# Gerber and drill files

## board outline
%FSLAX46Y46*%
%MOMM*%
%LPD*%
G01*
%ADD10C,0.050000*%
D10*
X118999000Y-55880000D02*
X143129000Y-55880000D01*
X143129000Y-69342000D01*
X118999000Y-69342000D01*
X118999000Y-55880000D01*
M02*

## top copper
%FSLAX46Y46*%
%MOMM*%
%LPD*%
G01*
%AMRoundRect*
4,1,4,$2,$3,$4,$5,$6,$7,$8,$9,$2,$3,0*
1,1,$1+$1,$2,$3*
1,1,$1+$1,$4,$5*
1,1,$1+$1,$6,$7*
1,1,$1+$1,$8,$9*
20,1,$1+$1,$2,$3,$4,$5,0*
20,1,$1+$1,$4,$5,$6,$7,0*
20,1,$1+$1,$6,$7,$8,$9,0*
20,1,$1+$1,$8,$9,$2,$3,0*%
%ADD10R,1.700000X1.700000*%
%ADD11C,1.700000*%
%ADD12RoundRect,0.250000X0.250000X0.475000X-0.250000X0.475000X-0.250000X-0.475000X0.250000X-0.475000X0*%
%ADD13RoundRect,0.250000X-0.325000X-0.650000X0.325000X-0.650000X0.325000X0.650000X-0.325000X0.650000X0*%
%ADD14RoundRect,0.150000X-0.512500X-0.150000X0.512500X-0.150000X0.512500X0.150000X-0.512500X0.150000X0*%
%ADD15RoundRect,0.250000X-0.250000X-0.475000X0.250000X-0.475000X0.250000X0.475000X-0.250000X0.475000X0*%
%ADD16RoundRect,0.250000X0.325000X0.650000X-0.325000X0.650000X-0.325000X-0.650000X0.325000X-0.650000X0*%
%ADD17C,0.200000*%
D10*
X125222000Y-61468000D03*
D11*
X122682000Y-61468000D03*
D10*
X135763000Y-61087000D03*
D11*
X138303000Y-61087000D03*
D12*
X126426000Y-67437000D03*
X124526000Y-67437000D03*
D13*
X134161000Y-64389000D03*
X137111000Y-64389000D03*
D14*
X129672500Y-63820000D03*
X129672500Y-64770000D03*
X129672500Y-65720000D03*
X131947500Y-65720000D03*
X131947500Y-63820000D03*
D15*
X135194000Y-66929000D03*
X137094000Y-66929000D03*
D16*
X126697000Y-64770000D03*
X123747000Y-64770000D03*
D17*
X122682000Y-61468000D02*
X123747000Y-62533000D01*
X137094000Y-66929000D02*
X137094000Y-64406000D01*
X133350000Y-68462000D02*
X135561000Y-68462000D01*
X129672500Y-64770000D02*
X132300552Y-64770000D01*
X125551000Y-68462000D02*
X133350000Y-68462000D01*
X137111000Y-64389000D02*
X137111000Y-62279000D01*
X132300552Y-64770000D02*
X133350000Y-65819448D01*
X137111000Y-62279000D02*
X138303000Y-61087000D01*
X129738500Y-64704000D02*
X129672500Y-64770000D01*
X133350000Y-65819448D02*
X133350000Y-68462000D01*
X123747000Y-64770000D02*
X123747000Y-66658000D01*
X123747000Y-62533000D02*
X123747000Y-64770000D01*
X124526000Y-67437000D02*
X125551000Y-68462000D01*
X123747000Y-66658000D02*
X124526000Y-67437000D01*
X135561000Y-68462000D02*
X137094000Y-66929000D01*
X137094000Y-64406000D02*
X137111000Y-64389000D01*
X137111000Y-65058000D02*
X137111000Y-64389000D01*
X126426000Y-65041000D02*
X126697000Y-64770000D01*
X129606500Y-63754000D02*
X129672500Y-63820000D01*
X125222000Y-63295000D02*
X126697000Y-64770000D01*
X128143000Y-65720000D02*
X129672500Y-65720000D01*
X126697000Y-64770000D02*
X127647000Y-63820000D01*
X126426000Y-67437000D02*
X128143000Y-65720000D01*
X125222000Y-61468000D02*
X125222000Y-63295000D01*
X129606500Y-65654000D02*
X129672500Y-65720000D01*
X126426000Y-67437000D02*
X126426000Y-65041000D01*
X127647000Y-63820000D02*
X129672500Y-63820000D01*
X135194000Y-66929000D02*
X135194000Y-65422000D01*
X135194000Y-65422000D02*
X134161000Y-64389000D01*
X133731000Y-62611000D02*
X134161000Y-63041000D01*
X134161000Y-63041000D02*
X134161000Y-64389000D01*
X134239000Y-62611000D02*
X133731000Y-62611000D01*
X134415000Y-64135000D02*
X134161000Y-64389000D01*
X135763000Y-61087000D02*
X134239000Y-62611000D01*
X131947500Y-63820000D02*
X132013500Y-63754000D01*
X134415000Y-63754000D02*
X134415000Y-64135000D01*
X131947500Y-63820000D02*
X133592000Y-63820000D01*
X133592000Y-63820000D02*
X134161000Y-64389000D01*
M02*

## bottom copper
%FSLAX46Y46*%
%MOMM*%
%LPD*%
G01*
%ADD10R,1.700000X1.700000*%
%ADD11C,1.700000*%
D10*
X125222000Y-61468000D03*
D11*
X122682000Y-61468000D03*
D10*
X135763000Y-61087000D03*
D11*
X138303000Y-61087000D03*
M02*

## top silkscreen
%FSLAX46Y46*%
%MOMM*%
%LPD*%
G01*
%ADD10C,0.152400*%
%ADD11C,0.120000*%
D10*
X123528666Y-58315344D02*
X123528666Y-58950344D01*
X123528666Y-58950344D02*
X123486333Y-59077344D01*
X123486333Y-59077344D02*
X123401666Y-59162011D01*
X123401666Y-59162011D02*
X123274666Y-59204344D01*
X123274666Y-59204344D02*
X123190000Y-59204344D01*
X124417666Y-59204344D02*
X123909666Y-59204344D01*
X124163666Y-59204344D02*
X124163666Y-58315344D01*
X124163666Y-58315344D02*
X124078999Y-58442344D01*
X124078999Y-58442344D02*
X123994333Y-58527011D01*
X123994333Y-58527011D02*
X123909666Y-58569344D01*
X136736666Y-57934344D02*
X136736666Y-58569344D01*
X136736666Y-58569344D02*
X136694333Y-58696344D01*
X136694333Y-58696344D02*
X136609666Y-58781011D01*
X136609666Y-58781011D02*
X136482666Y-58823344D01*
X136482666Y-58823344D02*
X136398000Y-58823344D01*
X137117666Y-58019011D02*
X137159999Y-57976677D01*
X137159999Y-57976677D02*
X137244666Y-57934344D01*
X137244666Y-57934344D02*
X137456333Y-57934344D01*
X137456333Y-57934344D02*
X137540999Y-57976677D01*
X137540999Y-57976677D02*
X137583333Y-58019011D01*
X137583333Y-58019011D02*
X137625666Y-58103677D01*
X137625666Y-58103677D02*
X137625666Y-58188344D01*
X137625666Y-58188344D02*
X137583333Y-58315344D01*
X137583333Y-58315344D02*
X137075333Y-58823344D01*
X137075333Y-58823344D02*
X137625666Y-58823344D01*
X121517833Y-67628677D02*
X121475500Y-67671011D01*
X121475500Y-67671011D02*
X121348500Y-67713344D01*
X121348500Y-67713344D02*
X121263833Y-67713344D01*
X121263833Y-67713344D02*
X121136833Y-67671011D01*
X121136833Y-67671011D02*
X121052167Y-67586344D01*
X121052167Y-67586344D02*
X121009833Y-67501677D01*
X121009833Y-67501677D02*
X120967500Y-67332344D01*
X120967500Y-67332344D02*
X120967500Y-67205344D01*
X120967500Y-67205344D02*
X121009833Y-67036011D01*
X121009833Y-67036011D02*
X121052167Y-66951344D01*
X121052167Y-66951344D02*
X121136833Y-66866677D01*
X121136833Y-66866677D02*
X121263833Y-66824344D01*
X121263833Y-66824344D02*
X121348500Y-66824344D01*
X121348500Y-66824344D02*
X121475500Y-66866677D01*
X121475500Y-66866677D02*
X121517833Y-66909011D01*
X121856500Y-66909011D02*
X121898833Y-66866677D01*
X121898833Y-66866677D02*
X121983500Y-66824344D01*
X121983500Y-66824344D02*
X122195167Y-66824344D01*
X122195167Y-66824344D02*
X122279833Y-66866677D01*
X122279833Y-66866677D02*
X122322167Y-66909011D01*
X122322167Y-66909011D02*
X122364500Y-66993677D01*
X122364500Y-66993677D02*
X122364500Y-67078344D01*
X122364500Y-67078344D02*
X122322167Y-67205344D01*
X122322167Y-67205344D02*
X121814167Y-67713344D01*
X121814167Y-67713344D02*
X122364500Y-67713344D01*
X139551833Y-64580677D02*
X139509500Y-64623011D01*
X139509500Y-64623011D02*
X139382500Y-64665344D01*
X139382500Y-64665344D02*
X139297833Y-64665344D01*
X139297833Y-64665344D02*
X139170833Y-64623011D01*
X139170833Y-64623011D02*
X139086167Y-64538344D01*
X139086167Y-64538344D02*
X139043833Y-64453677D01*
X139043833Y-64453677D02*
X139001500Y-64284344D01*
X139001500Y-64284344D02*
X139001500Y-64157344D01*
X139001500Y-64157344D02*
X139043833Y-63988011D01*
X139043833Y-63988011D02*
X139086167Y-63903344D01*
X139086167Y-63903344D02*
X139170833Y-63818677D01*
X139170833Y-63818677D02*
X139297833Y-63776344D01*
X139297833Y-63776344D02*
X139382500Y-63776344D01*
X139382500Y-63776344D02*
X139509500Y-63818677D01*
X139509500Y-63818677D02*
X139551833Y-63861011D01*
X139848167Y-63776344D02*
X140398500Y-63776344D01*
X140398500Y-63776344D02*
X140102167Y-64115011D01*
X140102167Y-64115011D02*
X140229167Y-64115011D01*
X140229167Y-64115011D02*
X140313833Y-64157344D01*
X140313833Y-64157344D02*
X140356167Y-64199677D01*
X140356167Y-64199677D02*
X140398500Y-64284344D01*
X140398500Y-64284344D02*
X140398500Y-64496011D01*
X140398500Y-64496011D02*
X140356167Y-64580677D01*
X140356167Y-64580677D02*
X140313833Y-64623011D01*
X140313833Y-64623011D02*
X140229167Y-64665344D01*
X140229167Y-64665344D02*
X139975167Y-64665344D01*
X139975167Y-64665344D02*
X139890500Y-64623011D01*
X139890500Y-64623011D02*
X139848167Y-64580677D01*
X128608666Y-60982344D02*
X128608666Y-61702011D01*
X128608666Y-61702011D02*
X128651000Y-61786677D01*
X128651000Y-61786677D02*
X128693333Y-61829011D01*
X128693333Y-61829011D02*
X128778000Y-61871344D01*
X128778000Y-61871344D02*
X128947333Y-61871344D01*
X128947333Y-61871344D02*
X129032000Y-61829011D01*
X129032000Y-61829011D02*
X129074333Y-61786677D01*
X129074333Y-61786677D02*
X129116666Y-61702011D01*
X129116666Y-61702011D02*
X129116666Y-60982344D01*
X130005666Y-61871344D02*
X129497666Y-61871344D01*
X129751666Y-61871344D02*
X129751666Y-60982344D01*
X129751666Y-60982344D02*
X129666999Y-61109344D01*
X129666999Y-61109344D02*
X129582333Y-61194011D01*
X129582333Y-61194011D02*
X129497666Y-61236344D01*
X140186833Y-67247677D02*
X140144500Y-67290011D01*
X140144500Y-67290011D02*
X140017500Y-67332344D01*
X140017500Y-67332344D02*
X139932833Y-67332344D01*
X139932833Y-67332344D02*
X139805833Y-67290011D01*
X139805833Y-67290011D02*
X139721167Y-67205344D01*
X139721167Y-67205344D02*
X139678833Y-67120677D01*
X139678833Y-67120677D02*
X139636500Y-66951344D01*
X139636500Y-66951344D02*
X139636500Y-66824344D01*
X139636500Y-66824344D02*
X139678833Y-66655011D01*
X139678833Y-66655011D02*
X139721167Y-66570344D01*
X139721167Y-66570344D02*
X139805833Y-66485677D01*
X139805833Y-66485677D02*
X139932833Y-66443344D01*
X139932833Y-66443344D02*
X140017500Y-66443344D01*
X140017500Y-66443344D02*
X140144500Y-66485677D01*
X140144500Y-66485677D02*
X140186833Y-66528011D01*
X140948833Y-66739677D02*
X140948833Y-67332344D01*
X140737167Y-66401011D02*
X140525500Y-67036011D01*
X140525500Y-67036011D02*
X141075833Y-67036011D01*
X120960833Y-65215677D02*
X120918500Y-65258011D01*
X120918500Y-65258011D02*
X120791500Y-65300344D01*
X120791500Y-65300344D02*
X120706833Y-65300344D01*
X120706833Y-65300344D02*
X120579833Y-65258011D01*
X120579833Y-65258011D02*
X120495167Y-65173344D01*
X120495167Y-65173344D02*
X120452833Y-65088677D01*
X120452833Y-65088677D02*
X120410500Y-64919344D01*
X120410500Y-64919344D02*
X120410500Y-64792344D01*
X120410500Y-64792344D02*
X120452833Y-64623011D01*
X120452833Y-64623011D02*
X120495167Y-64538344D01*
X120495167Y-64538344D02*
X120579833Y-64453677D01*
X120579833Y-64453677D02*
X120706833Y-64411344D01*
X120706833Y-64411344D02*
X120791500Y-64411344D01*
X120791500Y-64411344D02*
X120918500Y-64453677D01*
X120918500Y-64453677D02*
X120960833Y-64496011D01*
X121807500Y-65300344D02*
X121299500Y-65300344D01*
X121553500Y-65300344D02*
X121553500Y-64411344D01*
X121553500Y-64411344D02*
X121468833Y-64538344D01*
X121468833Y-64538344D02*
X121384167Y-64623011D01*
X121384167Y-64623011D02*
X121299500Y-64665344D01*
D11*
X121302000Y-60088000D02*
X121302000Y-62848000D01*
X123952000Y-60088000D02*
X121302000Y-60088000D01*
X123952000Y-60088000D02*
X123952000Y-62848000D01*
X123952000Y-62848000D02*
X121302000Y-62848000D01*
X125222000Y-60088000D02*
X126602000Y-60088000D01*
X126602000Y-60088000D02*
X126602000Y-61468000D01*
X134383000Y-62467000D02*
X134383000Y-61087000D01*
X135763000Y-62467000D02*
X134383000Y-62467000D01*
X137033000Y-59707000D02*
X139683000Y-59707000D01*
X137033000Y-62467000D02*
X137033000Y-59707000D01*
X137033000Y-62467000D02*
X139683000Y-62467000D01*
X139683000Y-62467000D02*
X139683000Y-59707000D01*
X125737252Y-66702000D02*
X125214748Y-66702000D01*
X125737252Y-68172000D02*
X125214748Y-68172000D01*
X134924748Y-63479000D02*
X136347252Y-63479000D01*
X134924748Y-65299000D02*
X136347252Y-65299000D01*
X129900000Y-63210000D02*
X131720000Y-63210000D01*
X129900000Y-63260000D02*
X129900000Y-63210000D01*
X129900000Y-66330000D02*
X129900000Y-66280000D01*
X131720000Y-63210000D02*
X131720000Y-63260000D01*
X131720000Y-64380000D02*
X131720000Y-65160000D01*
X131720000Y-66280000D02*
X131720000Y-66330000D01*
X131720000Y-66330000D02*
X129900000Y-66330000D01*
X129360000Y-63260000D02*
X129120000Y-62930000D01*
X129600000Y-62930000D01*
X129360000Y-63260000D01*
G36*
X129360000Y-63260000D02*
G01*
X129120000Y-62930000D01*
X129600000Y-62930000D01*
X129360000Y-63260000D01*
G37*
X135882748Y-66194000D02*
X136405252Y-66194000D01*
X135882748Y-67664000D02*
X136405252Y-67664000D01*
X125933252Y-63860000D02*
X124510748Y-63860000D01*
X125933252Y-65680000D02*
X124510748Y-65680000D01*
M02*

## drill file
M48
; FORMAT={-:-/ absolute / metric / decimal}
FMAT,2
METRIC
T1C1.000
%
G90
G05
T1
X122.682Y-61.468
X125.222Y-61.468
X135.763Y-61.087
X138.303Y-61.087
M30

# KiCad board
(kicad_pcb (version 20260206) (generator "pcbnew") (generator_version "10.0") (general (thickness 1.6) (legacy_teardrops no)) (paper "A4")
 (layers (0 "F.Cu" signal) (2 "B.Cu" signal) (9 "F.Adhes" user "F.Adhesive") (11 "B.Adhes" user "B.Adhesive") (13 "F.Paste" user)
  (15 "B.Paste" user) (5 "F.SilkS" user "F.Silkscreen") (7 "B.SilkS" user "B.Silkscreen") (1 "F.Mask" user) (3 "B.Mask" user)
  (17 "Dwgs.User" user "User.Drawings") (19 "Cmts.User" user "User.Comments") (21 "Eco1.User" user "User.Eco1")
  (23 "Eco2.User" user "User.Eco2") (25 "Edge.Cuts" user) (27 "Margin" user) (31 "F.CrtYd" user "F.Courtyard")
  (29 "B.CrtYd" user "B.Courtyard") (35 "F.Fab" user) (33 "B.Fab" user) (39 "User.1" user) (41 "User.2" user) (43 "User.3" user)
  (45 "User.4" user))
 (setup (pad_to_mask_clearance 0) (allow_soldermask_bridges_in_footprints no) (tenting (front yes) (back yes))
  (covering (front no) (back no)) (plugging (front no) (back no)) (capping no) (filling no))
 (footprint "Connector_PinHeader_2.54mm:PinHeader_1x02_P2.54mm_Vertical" (layer "F.Cu") (at 125.222 61.468 -90)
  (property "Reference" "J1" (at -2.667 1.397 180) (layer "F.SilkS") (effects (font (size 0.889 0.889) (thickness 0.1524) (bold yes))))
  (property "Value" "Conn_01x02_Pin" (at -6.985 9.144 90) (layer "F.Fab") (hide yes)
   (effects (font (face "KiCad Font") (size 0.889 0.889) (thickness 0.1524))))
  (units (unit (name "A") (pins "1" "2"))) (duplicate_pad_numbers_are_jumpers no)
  (fp_line (start -1.38 3.92) (end 1.38 3.92) (stroke (width 0.12) (type solid)) (layer "F.SilkS"))
  (fp_line (start -1.38 1.27) (end -1.38 3.92) (stroke (width 0.12) (type solid)) (layer "F.SilkS"))
  (fp_line (start -1.38 1.27) (end 1.38 1.27) (stroke (width 0.12) (type solid)) (layer "F.SilkS"))
  (fp_line (start 1.38 1.27) (end 1.38 3.92) (stroke (width 0.12) (type solid)) (layer "F.SilkS"))
  (fp_line (start -1.38 0) (end -1.38 -1.38) (stroke (width 0.12) (type solid)) (layer "F.SilkS"))
  (fp_line (start -1.38 -1.38) (end 0 -1.38) (stroke (width 0.12) (type solid)) (layer "F.SilkS"))
  (pad "1" thru_hole rect (at 0 0 270) (size 1.7 1.7) (drill 1) (layers "*.Cu" "*.Mask") (remove_unused_layers no) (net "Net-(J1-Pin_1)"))
  (pad "2" thru_hole circle (at 0 2.54 270) (size 1.7 1.7) (drill 1) (layers "*.Cu" "*.Mask") (remove_unused_layers no) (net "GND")))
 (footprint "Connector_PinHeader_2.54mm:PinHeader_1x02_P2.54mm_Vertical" (layer "F.Cu") (at 135.763 61.087 90)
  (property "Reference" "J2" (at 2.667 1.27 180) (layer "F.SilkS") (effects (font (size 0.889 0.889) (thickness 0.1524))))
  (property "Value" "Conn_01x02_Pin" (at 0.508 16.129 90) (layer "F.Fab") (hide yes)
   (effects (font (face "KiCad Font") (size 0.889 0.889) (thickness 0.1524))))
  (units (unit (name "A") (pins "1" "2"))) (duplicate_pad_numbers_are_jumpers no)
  (fp_line (start -1.38 -1.38) (end 0 -1.38) (stroke (width 0.12) (type solid)) (layer "F.SilkS"))
  (fp_line (start -1.38 0) (end -1.38 -1.38) (stroke (width 0.12) (type solid)) (layer "F.SilkS"))
  (fp_line (start 1.38 1.27) (end 1.38 3.92) (stroke (width 0.12) (type solid)) (layer "F.SilkS"))
  (fp_line (start -1.38 1.27) (end 1.38 1.27) (stroke (width 0.12) (type solid)) (layer "F.SilkS"))
  (fp_line (start -1.38 1.27) (end -1.38 3.92) (stroke (width 0.12) (type solid)) (layer "F.SilkS"))
  (fp_line (start -1.38 3.92) (end 1.38 3.92) (stroke (width 0.12) (type solid)) (layer "F.SilkS"))
  (pad "1" thru_hole rect (at 0 0 90) (size 1.7 1.7) (drill 1) (layers "*.Cu" "*.Mask") (remove_unused_layers no) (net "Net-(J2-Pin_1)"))
  (pad "2" thru_hole circle (at 0 2.54 90) (size 1.7 1.7) (drill 1) (layers "*.Cu" "*.Mask") (remove_unused_layers no) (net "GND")))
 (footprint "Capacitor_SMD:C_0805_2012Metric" (layer "F.Cu") (at 125.476 67.437 180)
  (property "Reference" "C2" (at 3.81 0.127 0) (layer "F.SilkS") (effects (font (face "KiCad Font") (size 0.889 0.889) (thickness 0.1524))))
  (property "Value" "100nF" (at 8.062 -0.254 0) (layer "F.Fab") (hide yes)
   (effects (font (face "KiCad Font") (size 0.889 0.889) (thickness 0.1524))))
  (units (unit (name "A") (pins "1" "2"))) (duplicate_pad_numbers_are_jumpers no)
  (fp_line (start -0.261252 0.735) (end 0.261252 0.735) (stroke (width 0.12) (type solid)) (layer "F.SilkS"))
  (fp_line (start -0.261252 -0.735) (end 0.261252 -0.735) (stroke (width 0.12) (type solid)) (layer "F.SilkS"))
  (pad "1" smd roundrect (at -0.95 0 180) (size 1 1.45) (layers "F.Cu" "F.Mask" "F.Paste") (roundrect_rratio 0.25) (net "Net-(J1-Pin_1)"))
  (pad "2" smd roundrect (at 0.95 0 180) (size 1 1.45) (layers "F.Cu" "F.Mask" "F.Paste") (roundrect_rratio 0.25) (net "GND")))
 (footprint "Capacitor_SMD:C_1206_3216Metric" (layer "F.Cu") (at 135.636 64.389)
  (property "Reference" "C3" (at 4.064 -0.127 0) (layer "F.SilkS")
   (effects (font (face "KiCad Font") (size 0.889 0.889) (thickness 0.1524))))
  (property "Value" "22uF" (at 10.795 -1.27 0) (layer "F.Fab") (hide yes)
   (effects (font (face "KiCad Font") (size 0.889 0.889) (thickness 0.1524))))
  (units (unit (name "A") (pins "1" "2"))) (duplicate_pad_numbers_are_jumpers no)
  (fp_line (start -0.711252 -0.91) (end 0.711252 -0.91) (stroke (width 0.12) (type solid)) (layer "F.SilkS"))
  (fp_line (start -0.711252 0.91) (end 0.711252 0.91) (stroke (width 0.12) (type solid)) (layer "F.SilkS"))
  (pad "1" smd roundrect (at -1.475 0) (size 1.15 1.8) (layers "F.Cu" "F.Mask" "F.Paste") (roundrect_rratio 0.217391) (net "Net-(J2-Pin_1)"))
  (pad "2" smd roundrect (at 1.475 0) (size 1.15 1.8) (layers "F.Cu" "F.Mask" "F.Paste") (roundrect_rratio 0.217391) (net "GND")))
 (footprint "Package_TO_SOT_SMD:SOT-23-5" (layer "F.Cu") (at 130.81 64.77)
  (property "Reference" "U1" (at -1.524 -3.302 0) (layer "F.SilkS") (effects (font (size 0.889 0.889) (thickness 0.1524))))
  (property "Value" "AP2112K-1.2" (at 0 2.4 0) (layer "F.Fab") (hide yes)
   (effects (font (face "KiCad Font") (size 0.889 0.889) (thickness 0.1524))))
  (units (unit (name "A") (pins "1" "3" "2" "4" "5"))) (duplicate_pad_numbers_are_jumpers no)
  (fp_line (start -0.91 -1.56) (end 0.91 -1.56) (stroke (width 0.12) (type solid)) (layer "F.SilkS"))
  (fp_line (start -0.91 -1.51) (end -0.91 -1.56) (stroke (width 0.12) (type solid)) (layer "F.SilkS"))
  (fp_line (start -0.91 1.56) (end -0.91 1.51) (stroke (width 0.12) (type solid)) (layer "F.SilkS"))
  (fp_line (start 0.91 -1.56) (end 0.91 -1.51) (stroke (width 0.12) (type solid)) (layer "F.SilkS"))
  (fp_line (start 0.91 -0.39) (end 0.91 0.39) (stroke (width 0.12) (type solid)) (layer "F.SilkS"))
  (fp_line (start 0.91 1.51) (end 0.91 1.56) (stroke (width 0.12) (type solid)) (layer "F.SilkS"))
  (fp_line (start 0.91 1.56) (end -0.91 1.56) (stroke (width 0.12) (type solid)) (layer "F.SilkS"))
  (fp_poly (pts (xy -1.45 -1.51) (xy -1.69 -1.84) (xy -1.21 -1.84)) (stroke (width 0.12) (type solid)) (fill yes) (layer "F.SilkS"))
  (pad "1" smd roundrect (at -1.1375 -0.95) (size 1.325 0.6) (layers "F.Cu" "F.Mask" "F.Paste") (roundrect_rratio 0.25)
   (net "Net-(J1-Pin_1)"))
  (pad "2" smd roundrect (at -1.1375 0) (size 1.325 0.6) (layers "F.Cu" "F.Mask" "F.Paste") (roundrect_rratio 0.25) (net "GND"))
  (pad "3" smd roundrect (at -1.1375 0.95) (size 1.325 0.6) (layers "F.Cu" "F.Mask" "F.Paste") (roundrect_rratio 0.25)
   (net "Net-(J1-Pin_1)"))
  (pad "4" smd roundrect (at 1.1375 0.95) (size 1.325 0.6) (layers "F.Cu" "F.Mask" "F.Paste") (roundrect_rratio 0.25)
   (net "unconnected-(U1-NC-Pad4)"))
  (pad "5" smd roundrect (at 1.1375 -0.95) (size 1.325 0.6) (layers "F.Cu" "F.Mask" "F.Paste") (roundrect_rratio 0.25)
   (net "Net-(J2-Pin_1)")))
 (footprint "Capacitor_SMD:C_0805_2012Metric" (layer "F.Cu") (at 136.144 66.929)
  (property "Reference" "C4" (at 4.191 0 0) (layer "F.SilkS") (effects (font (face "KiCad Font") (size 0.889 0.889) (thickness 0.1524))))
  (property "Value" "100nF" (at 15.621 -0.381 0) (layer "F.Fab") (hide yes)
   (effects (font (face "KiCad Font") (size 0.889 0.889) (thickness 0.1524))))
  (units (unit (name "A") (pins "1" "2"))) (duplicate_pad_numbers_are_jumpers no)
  (fp_line (start -0.261252 -0.735) (end 0.261252 -0.735) (stroke (width 0.12) (type solid)) (layer "F.SilkS"))
  (fp_line (start -0.261252 0.735) (end 0.261252 0.735) (stroke (width 0.12) (type solid)) (layer "F.SilkS"))
  (pad "1" smd roundrect (at -0.95 0) (size 1 1.45) (layers "F.Cu" "F.Mask" "F.Paste") (roundrect_rratio 0.25) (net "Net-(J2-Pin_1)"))
  (pad "2" smd roundrect (at 0.95 0) (size 1 1.45) (layers "F.Cu" "F.Mask" "F.Paste") (roundrect_rratio 0.25) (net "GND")))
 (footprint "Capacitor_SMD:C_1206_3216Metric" (layer "F.Cu") (at 125.222 64.77 180)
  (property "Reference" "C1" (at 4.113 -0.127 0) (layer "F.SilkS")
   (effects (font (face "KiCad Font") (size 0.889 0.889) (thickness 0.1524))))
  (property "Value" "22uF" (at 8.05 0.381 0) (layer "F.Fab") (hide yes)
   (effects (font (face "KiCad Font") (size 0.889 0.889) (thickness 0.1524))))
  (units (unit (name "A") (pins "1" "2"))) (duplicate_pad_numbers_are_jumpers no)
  (fp_line (start -0.711252 0.91) (end 0.711252 0.91) (stroke (width 0.12) (type solid)) (layer "F.SilkS"))
  (fp_line (start -0.711252 -0.91) (end 0.711252 -0.91) (stroke (width 0.12) (type solid)) (layer "F.SilkS"))
  (pad "1" smd roundrect (at -1.475 0 180) (size 1.15 1.8) (layers "F.Cu" "F.Mask" "F.Paste") (roundrect_rratio 0.217391)
   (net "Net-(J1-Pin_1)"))
  (pad "2" smd roundrect (at 1.475 0 180) (size 1.15 1.8) (layers "F.Cu" "F.Mask" "F.Paste") (roundrect_rratio 0.217391) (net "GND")))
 (gr_rect (start 118.999 55.88) (end 143.129 69.342) (stroke (width 0.05) (type default)) (fill no) (layer "Edge.Cuts"))
 (segment (start 122.682 61.468) (end 123.747 62.533) (width 0.2) (layer "F.Cu") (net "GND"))
 (segment (start 137.094 66.929) (end 137.094 64.406) (width 0.2) (layer "F.Cu") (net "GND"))
 (segment (start 133.35 68.462) (end 135.561 68.462) (width 0.2) (layer "F.Cu") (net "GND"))
 (segment (start 129.6725 64.77) (end 132.300552 64.77) (width 0.2) (layer "F.Cu") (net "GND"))
 (segment (start 125.551 68.462) (end 133.35 68.462) (width 0.2) (layer "F.Cu") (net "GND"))
 (segment (start 137.111 64.389) (end 137.111 62.279) (width 0.2) (layer "F.Cu") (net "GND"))
 (segment (start 132.300552 64.77) (end 133.35 65.819448) (width 0.2) (layer "F.Cu") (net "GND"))
 (segment (start 137.111 62.279) (end 138.303 61.087) (width 0.2) (layer "F.Cu") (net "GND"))
 (segment (start 129.7385 64.704) (end 129.6725 64.77) (width 0.2) (layer "F.Cu") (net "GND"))
 (segment (start 133.35 65.819448) (end 133.35 68.462) (width 0.2) (layer "F.Cu") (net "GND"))
 (segment (start 123.747 64.77) (end 123.747 66.658) (width 0.2) (layer "F.Cu") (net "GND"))
 (segment (start 123.747 62.533) (end 123.747 64.77) (width 0.2) (layer "F.Cu") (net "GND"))
 (segment (start 124.526 67.437) (end 125.551 68.462) (width 0.2) (layer "F.Cu") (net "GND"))
 (segment (start 123.747 66.658) (end 124.526 67.437) (width 0.2) (layer "F.Cu") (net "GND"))
 (segment (start 135.561 68.462) (end 137.094 66.929) (width 0.2) (layer "F.Cu") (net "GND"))
 (segment (start 137.094 64.406) (end 137.111 64.389) (width 0.2) (layer "F.Cu") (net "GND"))
 (segment (start 137.111 65.058) (end 137.111 64.389) (width 0.2) (layer "F.Cu") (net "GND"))
 (segment (start 126.426 65.041) (end 126.697 64.77) (width 0.2) (layer "F.Cu") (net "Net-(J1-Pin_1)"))
 (segment (start 129.6065 63.754) (end 129.6725 63.82) (width 0.2) (layer "F.Cu") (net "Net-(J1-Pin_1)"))
 (segment (start 125.222 63.295) (end 126.697 64.77) (width 0.2) (layer "F.Cu") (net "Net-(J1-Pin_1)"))
 (segment (start 128.143 65.72) (end 129.6725 65.72) (width 0.2) (layer "F.Cu") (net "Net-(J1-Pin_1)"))
 (segment (start 126.697 64.77) (end 127.647 63.82) (width 0.2) (layer "F.Cu") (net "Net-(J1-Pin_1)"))
 (segment (start 126.426 67.437) (end 128.143 65.72) (width 0.2) (layer "F.Cu") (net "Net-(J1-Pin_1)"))
 (segment (start 125.222 61.468) (end 125.222 63.295) (width 0.2) (layer "F.Cu") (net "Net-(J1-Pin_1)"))
 (segment (start 129.6065 65.654) (end 129.6725 65.72) (width 0.2) (layer "F.Cu") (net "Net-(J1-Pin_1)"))
 (segment (start 126.426 67.437) (end 126.426 65.041) (width 0.2) (layer "F.Cu") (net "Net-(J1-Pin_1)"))
 (segment (start 127.647 63.82) (end 129.6725 63.82) (width 0.2) (layer "F.Cu") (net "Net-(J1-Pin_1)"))
 (segment (start 135.194 66.929) (end 135.194 65.422) (width 0.2) (layer "F.Cu") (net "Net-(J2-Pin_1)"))
 (segment (start 135.194 65.422) (end 134.161 64.389) (width 0.2) (layer "F.Cu") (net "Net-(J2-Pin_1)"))
 (segment (start 133.731 62.611) (end 134.161 63.041) (width 0.2) (layer "F.Cu") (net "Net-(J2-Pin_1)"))
 (segment (start 134.161 63.041) (end 134.161 64.389) (width 0.2) (layer "F.Cu") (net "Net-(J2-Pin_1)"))
 (segment (start 134.239 62.611) (end 133.731 62.611) (width 0.2) (layer "F.Cu") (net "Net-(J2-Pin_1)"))
 (segment (start 134.415 64.135) (end 134.161 64.389) (width 0.2) (layer "F.Cu") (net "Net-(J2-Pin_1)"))
 (segment (start 135.763 61.087) (end 134.239 62.611) (width 0.2) (layer "F.Cu") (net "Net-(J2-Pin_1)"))
 (segment (start 131.9475 63.82) (end 132.0135 63.754) (width 0.2) (layer "F.Cu") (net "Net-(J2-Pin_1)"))
 (segment (start 134.415 63.754) (end 134.415 64.135) (width 0.2) (layer "F.Cu") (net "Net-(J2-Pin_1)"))
 (segment (start 131.9475 63.82) (end 133.592 63.82) (width 0.2) (layer "F.Cu") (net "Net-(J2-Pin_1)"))
 (segment (start 133.592 63.82) (end 134.161 64.389) (width 0.2) (layer "F.Cu") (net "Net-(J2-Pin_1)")))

